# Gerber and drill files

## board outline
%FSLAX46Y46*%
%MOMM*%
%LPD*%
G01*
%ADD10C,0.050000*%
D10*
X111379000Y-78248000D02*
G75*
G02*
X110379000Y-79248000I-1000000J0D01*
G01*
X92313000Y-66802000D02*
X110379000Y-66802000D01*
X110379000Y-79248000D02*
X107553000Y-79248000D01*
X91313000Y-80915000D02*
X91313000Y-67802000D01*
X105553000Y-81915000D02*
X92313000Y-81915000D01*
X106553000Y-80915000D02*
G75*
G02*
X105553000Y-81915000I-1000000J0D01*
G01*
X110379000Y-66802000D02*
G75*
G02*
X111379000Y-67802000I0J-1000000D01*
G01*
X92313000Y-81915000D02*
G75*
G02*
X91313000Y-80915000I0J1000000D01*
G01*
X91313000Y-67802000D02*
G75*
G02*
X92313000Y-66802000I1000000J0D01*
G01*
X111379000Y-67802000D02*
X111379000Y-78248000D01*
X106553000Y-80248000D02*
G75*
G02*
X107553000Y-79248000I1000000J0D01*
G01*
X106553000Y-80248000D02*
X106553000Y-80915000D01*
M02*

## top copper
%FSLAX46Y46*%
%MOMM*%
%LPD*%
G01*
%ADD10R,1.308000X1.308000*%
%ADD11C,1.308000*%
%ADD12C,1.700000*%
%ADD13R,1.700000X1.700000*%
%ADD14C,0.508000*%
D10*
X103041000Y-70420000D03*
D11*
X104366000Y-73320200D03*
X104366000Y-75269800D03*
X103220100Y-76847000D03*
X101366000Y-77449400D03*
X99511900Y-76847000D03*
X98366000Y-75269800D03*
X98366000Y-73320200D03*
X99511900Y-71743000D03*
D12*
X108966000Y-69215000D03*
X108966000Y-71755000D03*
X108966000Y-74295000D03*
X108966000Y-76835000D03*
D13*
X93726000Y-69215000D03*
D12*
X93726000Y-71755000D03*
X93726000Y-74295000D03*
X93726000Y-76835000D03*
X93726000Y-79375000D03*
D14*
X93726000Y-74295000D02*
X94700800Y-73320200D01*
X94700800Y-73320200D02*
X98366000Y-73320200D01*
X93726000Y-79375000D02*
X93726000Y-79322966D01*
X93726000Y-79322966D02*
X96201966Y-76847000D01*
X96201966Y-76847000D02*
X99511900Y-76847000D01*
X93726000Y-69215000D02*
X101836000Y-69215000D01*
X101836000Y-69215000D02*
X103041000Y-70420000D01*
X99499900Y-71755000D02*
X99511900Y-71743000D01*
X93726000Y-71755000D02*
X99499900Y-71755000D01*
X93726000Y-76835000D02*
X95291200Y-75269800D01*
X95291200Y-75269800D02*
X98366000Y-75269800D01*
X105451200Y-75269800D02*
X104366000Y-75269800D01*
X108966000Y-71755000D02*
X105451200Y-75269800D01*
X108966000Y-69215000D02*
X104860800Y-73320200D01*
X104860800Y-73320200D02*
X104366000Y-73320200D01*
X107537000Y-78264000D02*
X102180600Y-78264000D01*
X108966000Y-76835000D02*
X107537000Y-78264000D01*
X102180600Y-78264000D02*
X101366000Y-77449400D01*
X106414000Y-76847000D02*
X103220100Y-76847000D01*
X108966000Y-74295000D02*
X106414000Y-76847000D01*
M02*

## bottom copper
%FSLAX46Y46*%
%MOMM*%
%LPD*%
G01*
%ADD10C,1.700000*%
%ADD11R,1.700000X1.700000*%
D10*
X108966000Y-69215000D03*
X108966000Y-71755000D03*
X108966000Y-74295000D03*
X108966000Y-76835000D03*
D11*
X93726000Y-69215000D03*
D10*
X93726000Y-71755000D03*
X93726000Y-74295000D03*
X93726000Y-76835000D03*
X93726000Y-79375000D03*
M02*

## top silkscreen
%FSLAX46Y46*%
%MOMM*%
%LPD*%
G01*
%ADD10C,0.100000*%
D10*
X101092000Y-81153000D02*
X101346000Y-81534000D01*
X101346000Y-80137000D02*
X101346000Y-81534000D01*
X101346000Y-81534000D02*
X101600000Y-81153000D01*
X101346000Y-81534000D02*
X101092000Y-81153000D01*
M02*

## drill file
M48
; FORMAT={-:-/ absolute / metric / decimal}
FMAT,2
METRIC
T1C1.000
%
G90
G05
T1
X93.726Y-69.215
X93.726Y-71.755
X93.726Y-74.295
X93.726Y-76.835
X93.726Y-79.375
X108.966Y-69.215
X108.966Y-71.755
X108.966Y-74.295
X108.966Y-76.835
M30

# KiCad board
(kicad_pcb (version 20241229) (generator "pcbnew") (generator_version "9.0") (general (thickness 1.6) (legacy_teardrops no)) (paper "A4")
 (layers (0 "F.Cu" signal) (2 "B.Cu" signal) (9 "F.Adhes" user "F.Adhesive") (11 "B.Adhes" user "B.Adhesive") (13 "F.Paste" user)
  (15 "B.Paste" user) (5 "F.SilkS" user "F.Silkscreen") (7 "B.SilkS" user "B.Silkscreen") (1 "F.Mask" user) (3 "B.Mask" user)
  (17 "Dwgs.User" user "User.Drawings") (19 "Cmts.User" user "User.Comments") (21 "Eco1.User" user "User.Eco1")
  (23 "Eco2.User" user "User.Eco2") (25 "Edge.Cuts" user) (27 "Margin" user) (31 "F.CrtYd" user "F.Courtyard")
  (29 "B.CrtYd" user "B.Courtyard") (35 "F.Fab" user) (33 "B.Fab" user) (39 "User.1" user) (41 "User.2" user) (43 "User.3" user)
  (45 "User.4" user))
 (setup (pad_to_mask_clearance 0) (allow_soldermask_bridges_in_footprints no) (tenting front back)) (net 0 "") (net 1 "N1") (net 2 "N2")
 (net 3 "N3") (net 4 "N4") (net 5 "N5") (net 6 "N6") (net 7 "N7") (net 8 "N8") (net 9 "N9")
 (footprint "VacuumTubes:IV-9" (layer "F.Cu") (at 101.366 74.295 180)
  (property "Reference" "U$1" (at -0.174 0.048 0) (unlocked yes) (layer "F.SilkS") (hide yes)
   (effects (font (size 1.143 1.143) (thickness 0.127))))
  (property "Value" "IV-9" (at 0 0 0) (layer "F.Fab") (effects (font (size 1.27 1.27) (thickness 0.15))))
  (pad "1" connect rect (at -1.675 3.875 180) (size 1.308 1.308) (layers "F.Cu" "F.Mask") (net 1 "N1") (solder_mask_margin 0.1016)
   (thermal_bridge_angle 0))
  (pad "2" connect circle (at -3 0.9748 180) (size 1.308 1.308) (layers "F.Cu" "F.Mask") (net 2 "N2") (solder_mask_margin 0.1016)
   (thermal_bridge_angle 0))
  (pad "3" connect circle (at -3 -0.9748 180) (size 1.308 1.308) (layers "F.Cu" "F.Mask") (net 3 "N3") (solder_mask_margin 0.1016)
   (thermal_bridge_angle 0))
  (pad "4" connect circle (at -1.8541 -2.552 180) (size 1.308 1.308) (layers "F.Cu" "F.Mask") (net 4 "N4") (solder_mask_margin 0.1016)
   (thermal_bridge_angle 0))
  (pad "5" connect circle (at 0 -3.1544 180) (size 1.308 1.308) (layers "F.Cu" "F.Mask") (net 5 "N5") (solder_mask_margin 0.1016)
   (thermal_bridge_angle 0))
  (pad "6" connect circle (at 1.8541 -2.552 180) (size 1.308 1.308) (layers "F.Cu" "F.Mask") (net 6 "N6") (solder_mask_margin 0.1016)
   (thermal_bridge_angle 0))
  (pad "7" connect circle (at 3 -0.9748 180) (size 1.308 1.308) (layers "F.Cu" "F.Mask") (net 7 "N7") (solder_mask_margin 0.1016)
   (thermal_bridge_angle 0))
  (pad "8" connect circle (at 3 0.9748 180) (size 1.308 1.308) (layers "F.Cu" "F.Mask") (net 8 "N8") (solder_mask_margin 0.1016)
   (thermal_bridge_angle 0))
  (pad "9" connect circle (at 1.8541 2.552 180) (size 1.308 1.308) (layers "F.Cu" "F.Mask") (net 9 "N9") (solder_mask_margin 0.1016)
   (thermal_bridge_angle 0)))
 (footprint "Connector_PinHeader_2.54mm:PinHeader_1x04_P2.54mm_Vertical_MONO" (layer "B.Cu") (at 108.966 69.215 180)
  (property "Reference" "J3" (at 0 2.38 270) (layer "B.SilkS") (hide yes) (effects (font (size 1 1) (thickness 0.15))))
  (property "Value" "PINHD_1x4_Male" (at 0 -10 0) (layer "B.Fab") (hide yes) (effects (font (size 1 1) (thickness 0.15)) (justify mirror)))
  (pad "1" thru_hole circle (at 0 0 180) (size 1.7 1.7) (drill 1) (layers "*.Cu" "*.Mask") (remove_unused_layers no) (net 2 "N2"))
  (pad "2" thru_hole circle (at 0 -2.54 180) (size 1.7 1.7) (drill 1) (layers "*.Cu" "*.Mask") (remove_unused_layers no) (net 3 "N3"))
  (pad "3" thru_hole circle (at 0 -5.08 180) (size 1.7 1.7) (drill 1) (layers "*.Cu" "*.Mask") (remove_unused_layers no) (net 4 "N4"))
  (pad "4" thru_hole circle (at 0 -7.62 180) (size 1.7 1.7) (drill 1) (layers "*.Cu" "*.Mask") (remove_unused_layers no) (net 5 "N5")))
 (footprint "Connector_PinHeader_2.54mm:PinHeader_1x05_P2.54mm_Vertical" (layer "B.Cu") (at 93.726 69.215 180)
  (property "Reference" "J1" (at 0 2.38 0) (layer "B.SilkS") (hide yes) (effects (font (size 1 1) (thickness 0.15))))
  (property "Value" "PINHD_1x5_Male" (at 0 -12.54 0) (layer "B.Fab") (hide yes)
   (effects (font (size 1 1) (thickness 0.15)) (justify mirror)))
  (pad "1" thru_hole rect (at 0 0 180) (size 1.7 1.7) (drill 1) (layers "*.Cu" "*.Mask") (remove_unused_layers no) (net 1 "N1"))
  (pad "2" thru_hole circle (at 0 -2.54 180) (size 1.7 1.7) (drill 1) (layers "*.Cu" "*.Mask") (remove_unused_layers no) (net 9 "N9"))
  (pad "3" thru_hole circle (at 0 -5.08 180) (size 1.7 1.7) (drill 1) (layers "*.Cu" "*.Mask") (remove_unused_layers no) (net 8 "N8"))
  (pad "4" thru_hole circle (at 0 -7.62 180) (size 1.7 1.7) (drill 1) (layers "*.Cu" "*.Mask") (remove_unused_layers no) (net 7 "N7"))
  (pad "5" thru_hole circle (at 0 -10.16 180) (size 1.7 1.7) (drill 1) (layers "*.Cu" "*.Mask") (remove_unused_layers no) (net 6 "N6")))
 (gr_line (start 101.092 81.153) (end 101.346 81.534) (stroke (width 0.1) (type default)) (layer "F.SilkS"))
 (gr_line (start 101.346 80.137) (end 101.346 81.534) (stroke (width 0.1) (type default)) (layer "F.SilkS"))
 (gr_line (start 101.346 81.534) (end 101.6 81.153) (stroke (width 0.1) (type default)) (layer "F.SilkS"))
 (gr_line (start 101.346 81.534) (end 101.092 81.153) (stroke (width 0.1) (type default)) (layer "F.SilkS"))
 (gr_arc (start 111.379 78.248) (mid 111.086107 78.955107) (end 110.379 79.248) (stroke (width 0.05) (type default)) (layer "Edge.Cuts"))
 (gr_line (start 92.313 66.802) (end 110.379 66.802) (stroke (width 0.05) (type default)) (layer "Edge.Cuts"))
 (gr_line (start 110.379 79.248) (end 107.553 79.248) (stroke (width 0.05) (type default)) (layer "Edge.Cuts"))
 (gr_line (start 91.313 80.915) (end 91.313 67.802) (stroke (width 0.05) (type default)) (layer "Edge.Cuts"))
 (gr_line (start 105.553 81.915) (end 92.313 81.915) (stroke (width 0.05) (type default)) (layer "Edge.Cuts"))
 (gr_arc (start 106.553 80.915) (mid 106.260107 81.622107) (end 105.553 81.915) (stroke (width 0.05) (type default)) (layer "Edge.Cuts"))
 (gr_arc (start 110.379 66.802) (mid 111.086107 67.094893) (end 111.379 67.802) (stroke (width 0.05) (type default)) (layer "Edge.Cuts"))
 (gr_arc (start 92.313 81.915) (mid 91.605893 81.622107) (end 91.313 80.915) (stroke (width 0.05) (type default)) (layer "Edge.Cuts"))
 (gr_arc (start 91.313 67.802) (mid 91.605893 67.094893) (end 92.313 66.802) (stroke (width 0.05) (type default)) (layer "Edge.Cuts"))
 (gr_line (start 111.379 67.802) (end 111.379 78.248) (stroke (width 0.05) (type default)) (layer "Edge.Cuts"))
 (gr_arc (start 106.553 80.248) (mid 106.845893 79.540893) (end 107.553 79.248) (stroke (width 0.05) (type default)) (layer "Edge.Cuts"))
 (gr_line (start 106.553 80.248) (end 106.553 80.915) (stroke (width 0.05) (type default)) (layer "Edge.Cuts"))
 (segment (start 93.726 74.295) (end 94.7008 73.3202) (width 0.508) (layer "F.Cu") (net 8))
 (segment (start 94.7008 73.3202) (end 98.366 73.3202) (width 0.508) (layer "F.Cu") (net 8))
 (segment (start 93.726 79.375) (end 93.726 79.322966) (width 0.508) (layer "F.Cu") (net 6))
 (segment (start 93.726 79.322966) (end 96.201966 76.847) (width 0.508) (layer "F.Cu") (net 6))
 (segment (start 96.201966 76.847) (end 99.5119 76.847) (width 0.508) (layer "F.Cu") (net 6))
 (segment (start 93.726 69.215) (end 101.836 69.215) (width 0.508) (layer "F.Cu") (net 1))
 (segment (start 101.836 69.215) (end 103.041 70.42) (width 0.508) (layer "F.Cu") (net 1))
 (segment (start 99.4999 71.755) (end 99.5119 71.743) (width 0.508) (layer "F.Cu") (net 9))
 (segment (start 93.726 71.755) (end 99.4999 71.755) (width 0.508) (layer "F.Cu") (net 9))
 (segment (start 93.726 76.835) (end 95.2912 75.2698) (width 0.508) (layer "F.Cu") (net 7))
 (segment (start 95.2912 75.2698) (end 98.366 75.2698) (width 0.508) (layer "F.Cu") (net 7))
 (segment (start 105.4512 75.2698) (end 104.366 75.2698) (width 0.508) (layer "F.Cu") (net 3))
 (segment (start 108.966 71.755) (end 105.4512 75.2698) (width 0.508) (layer "F.Cu") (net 3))
 (segment (start 108.966 69.215) (end 104.8608 73.3202) (width 0.508) (layer "F.Cu") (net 2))
 (segment (start 104.8608 73.3202) (end 104.366 73.3202) (width 0.508) (layer "F.Cu") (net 2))
 (segment (start 107.537 78.264) (end 102.1806 78.264) (width 0.508) (layer "F.Cu") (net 5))
 (segment (start 108.966 76.835) (end 107.537 78.264) (width 0.508) (layer "F.Cu") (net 5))
 (segment (start 102.1806 78.264) (end 101.366 77.4494) (width 0.508) (layer "F.Cu") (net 5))
 (segment (start 106.414 76.847) (end 103.2201 76.847) (width 0.508) (layer "F.Cu") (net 4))
 (segment (start 108.966 74.295) (end 106.414 76.847) (width 0.508) (layer "F.Cu") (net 4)))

